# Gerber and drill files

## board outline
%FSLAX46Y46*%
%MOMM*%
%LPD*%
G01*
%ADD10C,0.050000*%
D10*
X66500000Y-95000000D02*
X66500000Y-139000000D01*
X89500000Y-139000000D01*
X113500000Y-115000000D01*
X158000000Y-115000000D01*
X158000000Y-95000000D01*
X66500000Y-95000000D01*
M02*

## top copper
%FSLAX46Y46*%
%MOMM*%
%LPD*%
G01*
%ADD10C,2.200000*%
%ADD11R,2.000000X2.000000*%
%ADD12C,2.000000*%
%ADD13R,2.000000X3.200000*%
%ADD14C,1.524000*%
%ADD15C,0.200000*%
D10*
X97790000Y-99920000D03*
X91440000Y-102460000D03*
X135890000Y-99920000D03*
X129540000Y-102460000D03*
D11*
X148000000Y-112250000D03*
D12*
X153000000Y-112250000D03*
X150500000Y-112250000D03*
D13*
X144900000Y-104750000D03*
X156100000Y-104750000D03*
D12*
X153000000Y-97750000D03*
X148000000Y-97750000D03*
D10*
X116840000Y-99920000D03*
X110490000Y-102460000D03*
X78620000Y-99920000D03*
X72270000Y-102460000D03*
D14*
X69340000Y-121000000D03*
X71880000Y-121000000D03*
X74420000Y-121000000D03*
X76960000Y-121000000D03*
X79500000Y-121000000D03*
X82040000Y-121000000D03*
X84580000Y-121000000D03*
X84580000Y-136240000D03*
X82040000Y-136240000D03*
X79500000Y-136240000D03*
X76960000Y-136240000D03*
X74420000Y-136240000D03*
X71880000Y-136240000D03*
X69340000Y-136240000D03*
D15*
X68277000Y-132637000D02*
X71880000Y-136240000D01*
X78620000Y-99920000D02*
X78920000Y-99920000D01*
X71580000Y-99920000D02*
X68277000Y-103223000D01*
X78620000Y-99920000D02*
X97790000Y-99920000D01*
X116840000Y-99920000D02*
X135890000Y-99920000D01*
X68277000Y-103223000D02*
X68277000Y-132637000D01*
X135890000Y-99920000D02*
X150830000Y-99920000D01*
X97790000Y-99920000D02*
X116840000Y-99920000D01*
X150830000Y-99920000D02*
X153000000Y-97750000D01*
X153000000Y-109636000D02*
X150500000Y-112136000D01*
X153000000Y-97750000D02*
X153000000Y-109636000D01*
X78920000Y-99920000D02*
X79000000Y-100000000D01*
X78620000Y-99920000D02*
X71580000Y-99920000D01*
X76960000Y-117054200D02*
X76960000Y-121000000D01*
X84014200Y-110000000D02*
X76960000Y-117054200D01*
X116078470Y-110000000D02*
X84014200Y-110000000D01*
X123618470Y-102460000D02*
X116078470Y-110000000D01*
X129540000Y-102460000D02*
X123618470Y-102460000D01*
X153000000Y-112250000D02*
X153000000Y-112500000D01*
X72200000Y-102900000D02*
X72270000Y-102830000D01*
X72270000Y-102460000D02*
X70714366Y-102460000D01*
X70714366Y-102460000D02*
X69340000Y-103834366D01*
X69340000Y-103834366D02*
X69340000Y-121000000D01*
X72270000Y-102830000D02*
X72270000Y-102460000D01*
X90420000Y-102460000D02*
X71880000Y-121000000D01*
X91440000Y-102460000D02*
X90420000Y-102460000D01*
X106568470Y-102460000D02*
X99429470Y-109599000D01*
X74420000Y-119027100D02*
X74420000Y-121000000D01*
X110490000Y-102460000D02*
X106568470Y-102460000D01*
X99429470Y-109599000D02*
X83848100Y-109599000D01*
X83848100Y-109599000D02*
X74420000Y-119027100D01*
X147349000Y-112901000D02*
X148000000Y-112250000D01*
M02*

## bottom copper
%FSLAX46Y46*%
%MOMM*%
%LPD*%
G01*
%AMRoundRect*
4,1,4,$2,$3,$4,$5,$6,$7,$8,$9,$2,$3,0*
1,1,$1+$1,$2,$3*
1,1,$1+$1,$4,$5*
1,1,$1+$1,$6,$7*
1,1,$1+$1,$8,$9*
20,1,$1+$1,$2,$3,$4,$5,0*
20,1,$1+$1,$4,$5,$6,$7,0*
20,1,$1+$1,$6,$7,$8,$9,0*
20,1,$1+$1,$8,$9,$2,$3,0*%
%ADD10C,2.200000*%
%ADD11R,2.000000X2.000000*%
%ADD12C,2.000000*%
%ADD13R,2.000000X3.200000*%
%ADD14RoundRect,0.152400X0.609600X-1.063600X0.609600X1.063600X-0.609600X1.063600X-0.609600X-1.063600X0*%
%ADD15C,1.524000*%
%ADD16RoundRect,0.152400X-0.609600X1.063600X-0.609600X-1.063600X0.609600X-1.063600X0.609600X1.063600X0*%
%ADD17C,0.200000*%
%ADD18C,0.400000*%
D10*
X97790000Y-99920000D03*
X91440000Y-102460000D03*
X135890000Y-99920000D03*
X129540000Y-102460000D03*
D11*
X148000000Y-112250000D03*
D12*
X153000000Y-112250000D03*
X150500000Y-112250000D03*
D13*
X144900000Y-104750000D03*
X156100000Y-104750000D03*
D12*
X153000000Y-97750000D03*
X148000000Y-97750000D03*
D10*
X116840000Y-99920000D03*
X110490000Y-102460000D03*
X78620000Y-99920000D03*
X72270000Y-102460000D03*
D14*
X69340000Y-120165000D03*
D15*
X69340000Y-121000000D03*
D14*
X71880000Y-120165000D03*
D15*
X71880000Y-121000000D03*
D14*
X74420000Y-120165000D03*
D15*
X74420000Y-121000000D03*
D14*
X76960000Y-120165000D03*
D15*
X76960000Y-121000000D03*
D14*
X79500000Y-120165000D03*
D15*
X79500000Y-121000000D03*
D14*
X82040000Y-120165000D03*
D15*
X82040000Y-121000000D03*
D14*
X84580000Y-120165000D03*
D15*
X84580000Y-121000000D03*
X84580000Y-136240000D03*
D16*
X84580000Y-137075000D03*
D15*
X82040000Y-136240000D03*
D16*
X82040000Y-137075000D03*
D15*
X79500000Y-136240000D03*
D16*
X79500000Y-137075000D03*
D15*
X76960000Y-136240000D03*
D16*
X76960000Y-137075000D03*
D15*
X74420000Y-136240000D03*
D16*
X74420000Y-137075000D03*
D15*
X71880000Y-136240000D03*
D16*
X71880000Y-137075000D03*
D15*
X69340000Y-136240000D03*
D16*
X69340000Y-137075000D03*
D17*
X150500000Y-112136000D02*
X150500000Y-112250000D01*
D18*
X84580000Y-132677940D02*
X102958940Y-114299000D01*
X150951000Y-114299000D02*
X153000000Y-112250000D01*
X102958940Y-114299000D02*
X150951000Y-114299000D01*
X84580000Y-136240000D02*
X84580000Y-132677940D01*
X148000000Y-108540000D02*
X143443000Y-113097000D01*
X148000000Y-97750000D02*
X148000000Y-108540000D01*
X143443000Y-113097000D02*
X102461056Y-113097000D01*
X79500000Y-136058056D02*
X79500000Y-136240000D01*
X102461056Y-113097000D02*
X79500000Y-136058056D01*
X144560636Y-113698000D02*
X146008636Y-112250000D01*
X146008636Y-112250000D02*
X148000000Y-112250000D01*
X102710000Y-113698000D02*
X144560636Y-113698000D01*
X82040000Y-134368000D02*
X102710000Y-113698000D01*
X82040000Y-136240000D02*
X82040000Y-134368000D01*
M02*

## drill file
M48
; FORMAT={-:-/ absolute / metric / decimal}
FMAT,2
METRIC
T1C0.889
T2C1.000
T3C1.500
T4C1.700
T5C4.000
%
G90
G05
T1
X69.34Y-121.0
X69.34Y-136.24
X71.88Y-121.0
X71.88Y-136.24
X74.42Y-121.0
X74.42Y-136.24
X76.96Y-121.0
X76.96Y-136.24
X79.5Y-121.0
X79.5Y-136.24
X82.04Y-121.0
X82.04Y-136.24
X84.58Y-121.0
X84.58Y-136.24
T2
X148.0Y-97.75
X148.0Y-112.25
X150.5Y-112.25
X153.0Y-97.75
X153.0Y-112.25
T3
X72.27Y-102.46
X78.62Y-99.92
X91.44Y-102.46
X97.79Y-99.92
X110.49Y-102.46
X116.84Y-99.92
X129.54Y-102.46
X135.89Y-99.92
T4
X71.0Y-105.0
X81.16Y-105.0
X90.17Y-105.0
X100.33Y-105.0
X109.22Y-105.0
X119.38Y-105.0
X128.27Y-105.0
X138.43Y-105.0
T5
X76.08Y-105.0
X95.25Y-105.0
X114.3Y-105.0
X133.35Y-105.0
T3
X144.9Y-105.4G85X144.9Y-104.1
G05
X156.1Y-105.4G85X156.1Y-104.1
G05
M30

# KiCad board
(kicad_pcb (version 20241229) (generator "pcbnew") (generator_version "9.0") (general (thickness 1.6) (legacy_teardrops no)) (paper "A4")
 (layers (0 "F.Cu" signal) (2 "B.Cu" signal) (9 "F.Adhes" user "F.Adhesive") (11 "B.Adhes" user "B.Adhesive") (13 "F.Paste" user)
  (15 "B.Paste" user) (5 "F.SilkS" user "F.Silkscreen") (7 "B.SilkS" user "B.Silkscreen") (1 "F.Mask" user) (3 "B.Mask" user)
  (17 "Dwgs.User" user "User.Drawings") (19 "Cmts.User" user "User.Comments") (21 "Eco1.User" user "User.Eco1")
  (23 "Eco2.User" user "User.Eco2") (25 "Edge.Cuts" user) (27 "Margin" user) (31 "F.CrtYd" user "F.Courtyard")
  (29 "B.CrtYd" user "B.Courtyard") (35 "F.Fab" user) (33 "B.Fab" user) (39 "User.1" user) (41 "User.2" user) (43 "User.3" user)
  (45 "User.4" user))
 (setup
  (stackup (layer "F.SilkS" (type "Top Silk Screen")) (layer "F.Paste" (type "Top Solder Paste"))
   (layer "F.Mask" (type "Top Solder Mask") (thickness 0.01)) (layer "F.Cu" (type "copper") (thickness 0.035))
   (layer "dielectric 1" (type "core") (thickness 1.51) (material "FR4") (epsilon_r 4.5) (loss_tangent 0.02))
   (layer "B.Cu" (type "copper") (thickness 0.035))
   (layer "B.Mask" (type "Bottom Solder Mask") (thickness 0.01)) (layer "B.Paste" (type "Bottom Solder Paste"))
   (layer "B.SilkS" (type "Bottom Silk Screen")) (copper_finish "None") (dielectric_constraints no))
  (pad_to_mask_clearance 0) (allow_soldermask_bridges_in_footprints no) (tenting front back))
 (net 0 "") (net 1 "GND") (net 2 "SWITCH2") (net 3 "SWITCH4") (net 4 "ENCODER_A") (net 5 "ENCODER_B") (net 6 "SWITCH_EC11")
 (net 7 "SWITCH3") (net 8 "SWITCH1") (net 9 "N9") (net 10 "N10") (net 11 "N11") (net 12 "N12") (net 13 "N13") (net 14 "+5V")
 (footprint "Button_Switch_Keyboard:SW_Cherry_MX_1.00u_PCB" (layer "F.Cu") (at 97.79 99.92)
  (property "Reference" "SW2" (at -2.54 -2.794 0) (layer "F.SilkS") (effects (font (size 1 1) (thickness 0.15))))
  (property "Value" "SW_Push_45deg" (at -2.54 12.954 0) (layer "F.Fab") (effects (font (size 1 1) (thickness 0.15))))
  (pad "" np_thru_hole circle (at -7.62 5.08) (size 1.7 1.7) (drill 1.7) (layers "*.Cu" "*.Mask"))
  (pad "" np_thru_hole circle (at -2.54 5.08) (size 4 4) (drill 4) (layers "*.Cu" "*.Mask"))
  (pad "" np_thru_hole circle (at 2.54 5.08) (size 1.7 1.7) (drill 1.7) (layers "*.Cu" "*.Mask"))
  (pad "1" thru_hole circle (at 0 0) (size 2.2 2.2) (drill 1.5) (layers "*.Cu" "*.Mask") (remove_unused_layers no) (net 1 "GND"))
  (pad "2" thru_hole circle (at -6.35 2.54) (size 2.2 2.2) (drill 1.5) (layers "*.Cu" "*.Mask") (remove_unused_layers no) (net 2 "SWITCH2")))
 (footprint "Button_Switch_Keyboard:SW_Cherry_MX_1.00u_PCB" (layer "F.Cu") (at 135.89 99.92)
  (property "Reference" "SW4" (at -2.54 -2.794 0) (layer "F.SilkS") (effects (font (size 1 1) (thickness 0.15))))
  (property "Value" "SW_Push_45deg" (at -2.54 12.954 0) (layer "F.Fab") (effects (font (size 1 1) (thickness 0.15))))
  (pad "" np_thru_hole circle (at -7.62 5.08) (size 1.7 1.7) (drill 1.7) (layers "*.Cu" "*.Mask"))
  (pad "" np_thru_hole circle (at -2.54 5.08) (size 4 4) (drill 4) (layers "*.Cu" "*.Mask"))
  (pad "" np_thru_hole circle (at 2.54 5.08) (size 1.7 1.7) (drill 1.7) (layers "*.Cu" "*.Mask"))
  (pad "1" thru_hole circle (at 0 0) (size 2.2 2.2) (drill 1.5) (layers "*.Cu" "*.Mask") (remove_unused_layers no) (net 1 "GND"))
  (pad "2" thru_hole circle (at -6.35 2.54) (size 2.2 2.2) (drill 1.5) (layers "*.Cu" "*.Mask") (remove_unused_layers no) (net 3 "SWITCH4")))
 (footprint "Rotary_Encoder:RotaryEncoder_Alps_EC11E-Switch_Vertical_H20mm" (layer "F.Cu") (at 148 112.25 90)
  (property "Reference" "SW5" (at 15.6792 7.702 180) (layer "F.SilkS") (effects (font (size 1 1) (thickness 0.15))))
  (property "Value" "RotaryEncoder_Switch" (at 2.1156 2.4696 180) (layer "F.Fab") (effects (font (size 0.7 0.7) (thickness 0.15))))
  (pad "A" thru_hole rect (at 0 0 90) (size 2 2) (drill 1) (layers "*.Cu" "*.Mask") (remove_unused_layers no) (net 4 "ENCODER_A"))
  (pad "B" thru_hole circle (at 0 5 90) (size 2 2) (drill 1) (layers "*.Cu" "*.Mask") (remove_unused_layers no) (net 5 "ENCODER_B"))
  (pad "C" thru_hole circle (at 0 2.5 90) (size 2 2) (drill 1) (layers "*.Cu" "*.Mask") (remove_unused_layers no) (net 1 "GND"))
  (pad "MP" thru_hole rect (at 7.5 -3.1 90) (size 3.2 2) (drill oval 2.8 1.5) (layers "*.Cu" "*.Mask") (remove_unused_layers no))
  (pad "MP" thru_hole rect (at 7.5 8.1 90) (size 3.2 2) (drill oval 2.8 1.5) (layers "*.Cu" "*.Mask") (remove_unused_layers no))
  (pad "S1" thru_hole circle (at 14.5 5 90) (size 2 2) (drill 1) (layers "*.Cu" "*.Mask") (remove_unused_layers no) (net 1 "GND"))
  (pad "S2" thru_hole circle (at 14.5 0 90) (size 2 2) (drill 1) (layers "*.Cu" "*.Mask") (remove_unused_layers no) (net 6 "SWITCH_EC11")))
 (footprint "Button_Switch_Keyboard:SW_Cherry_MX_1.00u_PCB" (layer "F.Cu") (at 116.84 99.92)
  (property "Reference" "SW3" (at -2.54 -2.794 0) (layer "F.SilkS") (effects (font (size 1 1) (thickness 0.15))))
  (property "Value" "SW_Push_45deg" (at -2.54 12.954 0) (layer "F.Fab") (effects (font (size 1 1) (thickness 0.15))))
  (pad "" np_thru_hole circle (at -7.62 5.08) (size 1.7 1.7) (drill 1.7) (layers "*.Cu" "*.Mask"))
  (pad "" np_thru_hole circle (at -2.54 5.08) (size 4 4) (drill 4) (layers "*.Cu" "*.Mask"))
  (pad "" np_thru_hole circle (at 2.54 5.08) (size 1.7 1.7) (drill 1.7) (layers "*.Cu" "*.Mask"))
  (pad "1" thru_hole circle (at 0 0) (size 2.2 2.2) (drill 1.5) (layers "*.Cu" "*.Mask") (remove_unused_layers no) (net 1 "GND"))
  (pad "2" thru_hole circle (at -6.35 2.54) (size 2.2 2.2) (drill 1.5) (layers "*.Cu" "*.Mask") (remove_unused_layers no) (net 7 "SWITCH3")))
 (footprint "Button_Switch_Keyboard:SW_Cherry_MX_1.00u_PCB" (layer "F.Cu") (at 78.62 99.92)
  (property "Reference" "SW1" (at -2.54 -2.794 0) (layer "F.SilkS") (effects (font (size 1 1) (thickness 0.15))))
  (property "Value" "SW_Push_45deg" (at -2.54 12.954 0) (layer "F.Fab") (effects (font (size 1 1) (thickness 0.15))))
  (pad "" np_thru_hole circle (at -7.62 5.08) (size 1.7 1.7) (drill 1.7) (layers "*.Cu" "*.Mask"))
  (pad "" np_thru_hole circle (at -2.54 5.08) (size 4 4) (drill 4) (layers "*.Cu" "*.Mask"))
  (pad "" np_thru_hole circle (at 2.54 5.08) (size 1.7 1.7) (drill 1.7) (layers "*.Cu" "*.Mask"))
  (pad "1" thru_hole circle (at 0 0) (size 2.2 2.2) (drill 1.5) (layers "*.Cu" "*.Mask") (remove_unused_layers no) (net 1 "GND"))
  (pad "2" thru_hole circle (at -6.35 2.54) (size 2.2 2.2) (drill 1.5) (layers "*.Cu" "*.Mask") (remove_unused_layers no) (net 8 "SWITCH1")))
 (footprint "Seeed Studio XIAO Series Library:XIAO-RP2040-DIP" (layer "B.Cu") (at 76.96 128.62 -90)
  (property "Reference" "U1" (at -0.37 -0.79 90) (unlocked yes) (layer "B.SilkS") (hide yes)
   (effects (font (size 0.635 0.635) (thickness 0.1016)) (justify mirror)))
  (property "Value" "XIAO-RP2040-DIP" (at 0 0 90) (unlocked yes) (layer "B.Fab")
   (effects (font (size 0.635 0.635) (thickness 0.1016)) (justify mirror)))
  (pad "1" smd roundrect (at -8.455 7.62 90) (size 2.432 1.524) (layers "B.Cu" "B.Mask") (roundrect_rratio 0.1) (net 8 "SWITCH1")
   (thermal_bridge_angle 45))
  (pad "1" thru_hole circle (at -7.62 7.62 90) (size 1.524 1.524) (drill 0.889) (layers "*.Cu" "*.Mask") (remove_unused_layers no)
   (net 8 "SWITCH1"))
  (pad "2" smd roundrect (at -8.455 5.08 90) (size 2.432 1.524) (layers "B.Cu" "B.Mask") (roundrect_rratio 0.1) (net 2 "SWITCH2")
   (thermal_bridge_angle 45))
  (pad "2" thru_hole circle (at -7.62 5.08 90) (size 1.524 1.524) (drill 0.889) (layers "*.Cu" "*.Mask") (remove_unused_layers no)
   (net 2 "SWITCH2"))
  (pad "3" smd roundrect (at -8.455 2.54 90) (size 2.432 1.524) (layers "B.Cu" "B.Mask") (roundrect_rratio 0.1) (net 7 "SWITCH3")
   (thermal_bridge_angle 45))
  (pad "3" thru_hole circle (at -7.62 2.54 90) (size 1.524 1.524) (drill 0.889) (layers "*.Cu" "*.Mask") (remove_unused_layers no)
   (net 7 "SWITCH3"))
  (pad "4" smd roundrect (at -8.455 0 90) (size 2.432 1.524) (layers "B.Cu" "B.Mask") (roundrect_rratio 0.1) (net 3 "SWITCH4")
   (thermal_bridge_angle 45))
  (pad "4" thru_hole circle (at -7.62 0 90) (size 1.524 1.524) (drill 0.889) (layers "*.Cu" "*.Mask") (remove_unused_layers no)
   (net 3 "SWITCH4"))
  (pad "5" smd roundrect (at -8.455 -2.54 90) (size 2.432 1.524) (layers "B.Cu" "B.Mask") (roundrect_rratio 0.1) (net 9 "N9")
   (thermal_bridge_angle 45))
  (pad "5" thru_hole circle (at -7.62 -2.54 90) (size 1.524 1.524) (drill 0.889) (layers "*.Cu" "*.Mask") (remove_unused_layers no)
   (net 9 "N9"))
  (pad "6" smd roundrect (at -8.455 -5.08 90) (size 2.432 1.524) (layers "B.Cu" "B.Mask") (roundrect_rratio 0.1) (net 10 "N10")
   (thermal_bridge_angle 45))
  (pad "6" thru_hole circle (at -7.62 -5.08 90) (size 1.524 1.524) (drill 0.889) (layers "*.Cu" "*.Mask") (remove_unused_layers no)
   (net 10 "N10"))
  (pad "7" smd roundrect (at -8.455 -7.62 90) (size 2.432 1.524) (layers "B.Cu" "B.Mask") (roundrect_rratio 0.1) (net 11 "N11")
   (thermal_bridge_angle 45))
  (pad "7" thru_hole circle (at -7.62 -7.62 90) (size 1.524 1.524) (drill 0.889) (layers "*.Cu" "*.Mask") (remove_unused_layers no)
   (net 11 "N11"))
  (pad "8" thru_hole circle (at 7.62 -7.62 270) (size 1.524 1.524) (drill 0.889) (layers "*.Cu" "*.Mask") (remove_unused_layers no)
   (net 5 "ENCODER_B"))
  (pad "8" smd roundrect (at 8.455 -7.62 270) (size 2.432 1.524) (layers "B.Cu" "B.Mask") (roundrect_rratio 0.1) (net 5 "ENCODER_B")
   (thermal_bridge_angle 45))
  (pad "9" thru_hole circle (at 7.62 -5.08 270) (size 1.524 1.524) (drill 0.889) (layers "*.Cu" "*.Mask") (remove_unused_layers no)
   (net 4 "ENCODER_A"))
  (pad "9" smd roundrect (at 8.455 -5.08 270) (size 2.432 1.524) (layers "B.Cu" "B.Mask") (roundrect_rratio 0.1) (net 4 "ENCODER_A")
   (thermal_bridge_angle 45))
  (pad "10" thru_hole circle (at 7.62 -2.54 270) (size 1.524 1.524) (drill 0.889) (layers "*.Cu" "*.Mask") (remove_unused_layers no)
   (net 6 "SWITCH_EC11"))
  (pad "10" smd roundrect (at 8.455 -2.54 270) (size 2.432 1.524) (layers "B.Cu" "B.Mask") (roundrect_rratio 0.1) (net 6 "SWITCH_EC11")
   (thermal_bridge_angle 45))
  (pad "11" thru_hole circle (at 7.62 0 270) (size 1.524 1.524) (drill 0.889) (layers "*.Cu" "*.Mask") (remove_unused_layers no)
   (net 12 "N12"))
  (pad "11" smd roundrect (at 8.455 0 270) (size 2.432 1.524) (layers "B.Cu" "B.Mask") (roundrect_rratio 0.1) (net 12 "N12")
   (thermal_bridge_angle 45))
  (pad "12" thru_hole circle (at 7.62 2.54 270) (size 1.524 1.524) (drill 0.889) (layers "*.Cu" "*.Mask") (remove_unused_layers no)
   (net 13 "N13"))
  (pad "12" smd roundrect (at 8.455 2.54 270) (size 2.432 1.524) (layers "B.Cu" "B.Mask") (roundrect_rratio 0.1) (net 13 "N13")
   (thermal_bridge_angle 45))
  (pad "13" thru_hole circle (at 7.62 5.08 270) (size 1.524 1.524) (drill 0.889) (layers "*.Cu" "*.Mask") (remove_unused_layers no)
   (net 1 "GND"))
  (pad "13" smd roundrect (at 8.455 5.08 270) (size 2.432 1.524) (layers "B.Cu" "B.Mask") (roundrect_rratio 0.1) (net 1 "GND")
   (thermal_bridge_angle 45))
  (pad "14" thru_hole circle (at 7.62 7.62 270) (size 1.524 1.524) (drill 0.889) (layers "*.Cu" "*.Mask") (remove_unused_layers no)
   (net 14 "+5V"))
  (pad "14" smd roundrect (at 8.455 7.62 270) (size 2.432 1.524) (layers "B.Cu" "B.Mask") (roundrect_rratio 0.1) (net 14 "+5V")
   (thermal_bridge_angle 45)))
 (gr_poly
  (pts (xy 66.5 95) (xy 66.5 139) (xy 89.5 139) (xy 113.5 115) (xy 158 115) (xy 158 95)) (stroke (width 0.05) (type solid)) (fill no)
  (layer "Edge.Cuts"))
 (segment (start 68.277 132.637) (end 71.88 136.24) (width 0.2) (layer "F.Cu") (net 1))
 (segment (start 78.62 99.92) (end 78.92 99.92) (width 0.2) (layer "F.Cu") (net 1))
 (segment (start 71.58 99.92) (end 68.277 103.223) (width 0.2) (layer "F.Cu") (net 1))
 (segment (start 78.62 99.92) (end 97.79 99.92) (width 0.2) (layer "F.Cu") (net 1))
 (segment (start 116.84 99.92) (end 135.89 99.92) (width 0.2) (layer "F.Cu") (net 1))
 (segment (start 68.277 103.223) (end 68.277 132.637) (width 0.2) (layer "F.Cu") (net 1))
 (segment (start 135.89 99.92) (end 150.83 99.92) (width 0.2) (layer "F.Cu") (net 1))
 (segment (start 97.79 99.92) (end 116.84 99.92) (width 0.2) (layer "F.Cu") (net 1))
 (segment (start 150.83 99.92) (end 153 97.75) (width 0.2) (layer "F.Cu") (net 1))
 (segment (start 153 109.636) (end 150.5 112.136) (width 0.2) (layer "F.Cu") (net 1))
 (segment (start 153 97.75) (end 153 109.636) (width 0.2) (layer "F.Cu") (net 1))
 (segment (start 78.92 99.92) (end 79 100) (width 0.2) (layer "F.Cu") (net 1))
 (segment (start 78.62 99.92) (end 71.58 99.92) (width 0.2) (layer "F.Cu") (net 1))
 (segment (start 150.5 112.136) (end 150.5 112.25) (width 0.2) (layer "B.Cu") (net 1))
 (segment (start 76.96 117.0542) (end 76.96 121) (width 0.2) (layer "F.Cu") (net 3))
 (segment (start 84.0142 110) (end 76.96 117.0542) (width 0.2) (layer "F.Cu") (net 3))
 (segment (start 116.07847 110) (end 84.0142 110) (width 0.2) (layer "F.Cu") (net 3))
 (segment (start 123.61847 102.46) (end 116.07847 110) (width 0.2) (layer "F.Cu") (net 3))
 (segment (start 129.54 102.46) (end 123.61847 102.46) (width 0.2) (layer "F.Cu") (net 3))
 (segment (start 153 112.25) (end 153 112.5) (width 0.2) (layer "F.Cu") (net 5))
 (segment (start 84.58 132.67794) (end 102.95894 114.299) (width 0.4) (layer "B.Cu") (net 5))
 (segment (start 150.951 114.299) (end 153 112.25) (width 0.4) (layer "B.Cu") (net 5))
 (segment (start 102.95894 114.299) (end 150.951 114.299) (width 0.4) (layer "B.Cu") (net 5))
 (segment (start 84.58 136.24) (end 84.58 132.67794) (width 0.4) (layer "B.Cu") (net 5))
 (segment (start 72.2 102.9) (end 72.27 102.83) (width 0.2) (layer "F.Cu") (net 8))
 (segment (start 72.27 102.46) (end 70.714366 102.46) (width 0.2) (layer "F.Cu") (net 8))
 (segment (start 70.714366 102.46) (end 69.34 103.834366) (width 0.2) (layer "F.Cu") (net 8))
 (segment (start 69.34 103.834366) (end 69.34 121) (width 0.2) (layer "F.Cu") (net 8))
 (segment (start 72.27 102.83) (end 72.27 102.46) (width 0.2) (layer "F.Cu") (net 8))
 (segment (start 90.42 102.46) (end 71.88 121) (width 0.2) (layer "F.Cu") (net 2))
 (segment (start 91.44 102.46) (end 90.42 102.46) (width 0.2) (layer "F.Cu") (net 2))
 (segment (start 106.56847 102.46) (end 99.42947 109.599) (width 0.2) (layer "F.Cu") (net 7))
 (segment (start 74.42 119.0271) (end 74.42 121) (width 0.2) (layer "F.Cu") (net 7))
 (segment (start 110.49 102.46) (end 106.56847 102.46) (width 0.2) (layer "F.Cu") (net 7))
 (segment (start 99.42947 109.599) (end 83.8481 109.599) (width 0.2) (layer "F.Cu") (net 7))
 (segment (start 83.8481 109.599) (end 74.42 119.0271) (width 0.2) (layer "F.Cu") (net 7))
 (segment (start 148 108.54) (end 143.443 113.097) (width 0.4) (layer "B.Cu") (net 6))
 (segment (start 148 97.75) (end 148 108.54) (width 0.4) (layer "B.Cu") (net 6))
 (segment (start 143.443 113.097) (end 102.461056 113.097) (width 0.4) (layer "B.Cu") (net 6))
 (segment (start 79.5 136.058056) (end 79.5 136.24) (width 0.4) (layer "B.Cu") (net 6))
 (segment (start 102.461056 113.097) (end 79.5 136.058056) (width 0.4) (layer "B.Cu") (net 6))
 (segment (start 147.349 112.901) (end 148 112.25) (width 0.2) (layer "F.Cu") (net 4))
 (segment (start 144.560636 113.698) (end 146.008636 112.25) (width 0.4) (layer "B.Cu") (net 4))
 (segment (start 146.008636 112.25) (end 148 112.25) (width 0.4) (layer "B.Cu") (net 4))
 (segment (start 102.71 113.698) (end 144.560636 113.698) (width 0.4) (layer "B.Cu") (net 4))
 (segment (start 82.04 134.368) (end 102.71 113.698) (width 0.4) (layer "B.Cu") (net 4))
 (segment (start 82.04 136.24) (end 82.04 134.368) (width 0.4) (layer "B.Cu") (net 4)))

